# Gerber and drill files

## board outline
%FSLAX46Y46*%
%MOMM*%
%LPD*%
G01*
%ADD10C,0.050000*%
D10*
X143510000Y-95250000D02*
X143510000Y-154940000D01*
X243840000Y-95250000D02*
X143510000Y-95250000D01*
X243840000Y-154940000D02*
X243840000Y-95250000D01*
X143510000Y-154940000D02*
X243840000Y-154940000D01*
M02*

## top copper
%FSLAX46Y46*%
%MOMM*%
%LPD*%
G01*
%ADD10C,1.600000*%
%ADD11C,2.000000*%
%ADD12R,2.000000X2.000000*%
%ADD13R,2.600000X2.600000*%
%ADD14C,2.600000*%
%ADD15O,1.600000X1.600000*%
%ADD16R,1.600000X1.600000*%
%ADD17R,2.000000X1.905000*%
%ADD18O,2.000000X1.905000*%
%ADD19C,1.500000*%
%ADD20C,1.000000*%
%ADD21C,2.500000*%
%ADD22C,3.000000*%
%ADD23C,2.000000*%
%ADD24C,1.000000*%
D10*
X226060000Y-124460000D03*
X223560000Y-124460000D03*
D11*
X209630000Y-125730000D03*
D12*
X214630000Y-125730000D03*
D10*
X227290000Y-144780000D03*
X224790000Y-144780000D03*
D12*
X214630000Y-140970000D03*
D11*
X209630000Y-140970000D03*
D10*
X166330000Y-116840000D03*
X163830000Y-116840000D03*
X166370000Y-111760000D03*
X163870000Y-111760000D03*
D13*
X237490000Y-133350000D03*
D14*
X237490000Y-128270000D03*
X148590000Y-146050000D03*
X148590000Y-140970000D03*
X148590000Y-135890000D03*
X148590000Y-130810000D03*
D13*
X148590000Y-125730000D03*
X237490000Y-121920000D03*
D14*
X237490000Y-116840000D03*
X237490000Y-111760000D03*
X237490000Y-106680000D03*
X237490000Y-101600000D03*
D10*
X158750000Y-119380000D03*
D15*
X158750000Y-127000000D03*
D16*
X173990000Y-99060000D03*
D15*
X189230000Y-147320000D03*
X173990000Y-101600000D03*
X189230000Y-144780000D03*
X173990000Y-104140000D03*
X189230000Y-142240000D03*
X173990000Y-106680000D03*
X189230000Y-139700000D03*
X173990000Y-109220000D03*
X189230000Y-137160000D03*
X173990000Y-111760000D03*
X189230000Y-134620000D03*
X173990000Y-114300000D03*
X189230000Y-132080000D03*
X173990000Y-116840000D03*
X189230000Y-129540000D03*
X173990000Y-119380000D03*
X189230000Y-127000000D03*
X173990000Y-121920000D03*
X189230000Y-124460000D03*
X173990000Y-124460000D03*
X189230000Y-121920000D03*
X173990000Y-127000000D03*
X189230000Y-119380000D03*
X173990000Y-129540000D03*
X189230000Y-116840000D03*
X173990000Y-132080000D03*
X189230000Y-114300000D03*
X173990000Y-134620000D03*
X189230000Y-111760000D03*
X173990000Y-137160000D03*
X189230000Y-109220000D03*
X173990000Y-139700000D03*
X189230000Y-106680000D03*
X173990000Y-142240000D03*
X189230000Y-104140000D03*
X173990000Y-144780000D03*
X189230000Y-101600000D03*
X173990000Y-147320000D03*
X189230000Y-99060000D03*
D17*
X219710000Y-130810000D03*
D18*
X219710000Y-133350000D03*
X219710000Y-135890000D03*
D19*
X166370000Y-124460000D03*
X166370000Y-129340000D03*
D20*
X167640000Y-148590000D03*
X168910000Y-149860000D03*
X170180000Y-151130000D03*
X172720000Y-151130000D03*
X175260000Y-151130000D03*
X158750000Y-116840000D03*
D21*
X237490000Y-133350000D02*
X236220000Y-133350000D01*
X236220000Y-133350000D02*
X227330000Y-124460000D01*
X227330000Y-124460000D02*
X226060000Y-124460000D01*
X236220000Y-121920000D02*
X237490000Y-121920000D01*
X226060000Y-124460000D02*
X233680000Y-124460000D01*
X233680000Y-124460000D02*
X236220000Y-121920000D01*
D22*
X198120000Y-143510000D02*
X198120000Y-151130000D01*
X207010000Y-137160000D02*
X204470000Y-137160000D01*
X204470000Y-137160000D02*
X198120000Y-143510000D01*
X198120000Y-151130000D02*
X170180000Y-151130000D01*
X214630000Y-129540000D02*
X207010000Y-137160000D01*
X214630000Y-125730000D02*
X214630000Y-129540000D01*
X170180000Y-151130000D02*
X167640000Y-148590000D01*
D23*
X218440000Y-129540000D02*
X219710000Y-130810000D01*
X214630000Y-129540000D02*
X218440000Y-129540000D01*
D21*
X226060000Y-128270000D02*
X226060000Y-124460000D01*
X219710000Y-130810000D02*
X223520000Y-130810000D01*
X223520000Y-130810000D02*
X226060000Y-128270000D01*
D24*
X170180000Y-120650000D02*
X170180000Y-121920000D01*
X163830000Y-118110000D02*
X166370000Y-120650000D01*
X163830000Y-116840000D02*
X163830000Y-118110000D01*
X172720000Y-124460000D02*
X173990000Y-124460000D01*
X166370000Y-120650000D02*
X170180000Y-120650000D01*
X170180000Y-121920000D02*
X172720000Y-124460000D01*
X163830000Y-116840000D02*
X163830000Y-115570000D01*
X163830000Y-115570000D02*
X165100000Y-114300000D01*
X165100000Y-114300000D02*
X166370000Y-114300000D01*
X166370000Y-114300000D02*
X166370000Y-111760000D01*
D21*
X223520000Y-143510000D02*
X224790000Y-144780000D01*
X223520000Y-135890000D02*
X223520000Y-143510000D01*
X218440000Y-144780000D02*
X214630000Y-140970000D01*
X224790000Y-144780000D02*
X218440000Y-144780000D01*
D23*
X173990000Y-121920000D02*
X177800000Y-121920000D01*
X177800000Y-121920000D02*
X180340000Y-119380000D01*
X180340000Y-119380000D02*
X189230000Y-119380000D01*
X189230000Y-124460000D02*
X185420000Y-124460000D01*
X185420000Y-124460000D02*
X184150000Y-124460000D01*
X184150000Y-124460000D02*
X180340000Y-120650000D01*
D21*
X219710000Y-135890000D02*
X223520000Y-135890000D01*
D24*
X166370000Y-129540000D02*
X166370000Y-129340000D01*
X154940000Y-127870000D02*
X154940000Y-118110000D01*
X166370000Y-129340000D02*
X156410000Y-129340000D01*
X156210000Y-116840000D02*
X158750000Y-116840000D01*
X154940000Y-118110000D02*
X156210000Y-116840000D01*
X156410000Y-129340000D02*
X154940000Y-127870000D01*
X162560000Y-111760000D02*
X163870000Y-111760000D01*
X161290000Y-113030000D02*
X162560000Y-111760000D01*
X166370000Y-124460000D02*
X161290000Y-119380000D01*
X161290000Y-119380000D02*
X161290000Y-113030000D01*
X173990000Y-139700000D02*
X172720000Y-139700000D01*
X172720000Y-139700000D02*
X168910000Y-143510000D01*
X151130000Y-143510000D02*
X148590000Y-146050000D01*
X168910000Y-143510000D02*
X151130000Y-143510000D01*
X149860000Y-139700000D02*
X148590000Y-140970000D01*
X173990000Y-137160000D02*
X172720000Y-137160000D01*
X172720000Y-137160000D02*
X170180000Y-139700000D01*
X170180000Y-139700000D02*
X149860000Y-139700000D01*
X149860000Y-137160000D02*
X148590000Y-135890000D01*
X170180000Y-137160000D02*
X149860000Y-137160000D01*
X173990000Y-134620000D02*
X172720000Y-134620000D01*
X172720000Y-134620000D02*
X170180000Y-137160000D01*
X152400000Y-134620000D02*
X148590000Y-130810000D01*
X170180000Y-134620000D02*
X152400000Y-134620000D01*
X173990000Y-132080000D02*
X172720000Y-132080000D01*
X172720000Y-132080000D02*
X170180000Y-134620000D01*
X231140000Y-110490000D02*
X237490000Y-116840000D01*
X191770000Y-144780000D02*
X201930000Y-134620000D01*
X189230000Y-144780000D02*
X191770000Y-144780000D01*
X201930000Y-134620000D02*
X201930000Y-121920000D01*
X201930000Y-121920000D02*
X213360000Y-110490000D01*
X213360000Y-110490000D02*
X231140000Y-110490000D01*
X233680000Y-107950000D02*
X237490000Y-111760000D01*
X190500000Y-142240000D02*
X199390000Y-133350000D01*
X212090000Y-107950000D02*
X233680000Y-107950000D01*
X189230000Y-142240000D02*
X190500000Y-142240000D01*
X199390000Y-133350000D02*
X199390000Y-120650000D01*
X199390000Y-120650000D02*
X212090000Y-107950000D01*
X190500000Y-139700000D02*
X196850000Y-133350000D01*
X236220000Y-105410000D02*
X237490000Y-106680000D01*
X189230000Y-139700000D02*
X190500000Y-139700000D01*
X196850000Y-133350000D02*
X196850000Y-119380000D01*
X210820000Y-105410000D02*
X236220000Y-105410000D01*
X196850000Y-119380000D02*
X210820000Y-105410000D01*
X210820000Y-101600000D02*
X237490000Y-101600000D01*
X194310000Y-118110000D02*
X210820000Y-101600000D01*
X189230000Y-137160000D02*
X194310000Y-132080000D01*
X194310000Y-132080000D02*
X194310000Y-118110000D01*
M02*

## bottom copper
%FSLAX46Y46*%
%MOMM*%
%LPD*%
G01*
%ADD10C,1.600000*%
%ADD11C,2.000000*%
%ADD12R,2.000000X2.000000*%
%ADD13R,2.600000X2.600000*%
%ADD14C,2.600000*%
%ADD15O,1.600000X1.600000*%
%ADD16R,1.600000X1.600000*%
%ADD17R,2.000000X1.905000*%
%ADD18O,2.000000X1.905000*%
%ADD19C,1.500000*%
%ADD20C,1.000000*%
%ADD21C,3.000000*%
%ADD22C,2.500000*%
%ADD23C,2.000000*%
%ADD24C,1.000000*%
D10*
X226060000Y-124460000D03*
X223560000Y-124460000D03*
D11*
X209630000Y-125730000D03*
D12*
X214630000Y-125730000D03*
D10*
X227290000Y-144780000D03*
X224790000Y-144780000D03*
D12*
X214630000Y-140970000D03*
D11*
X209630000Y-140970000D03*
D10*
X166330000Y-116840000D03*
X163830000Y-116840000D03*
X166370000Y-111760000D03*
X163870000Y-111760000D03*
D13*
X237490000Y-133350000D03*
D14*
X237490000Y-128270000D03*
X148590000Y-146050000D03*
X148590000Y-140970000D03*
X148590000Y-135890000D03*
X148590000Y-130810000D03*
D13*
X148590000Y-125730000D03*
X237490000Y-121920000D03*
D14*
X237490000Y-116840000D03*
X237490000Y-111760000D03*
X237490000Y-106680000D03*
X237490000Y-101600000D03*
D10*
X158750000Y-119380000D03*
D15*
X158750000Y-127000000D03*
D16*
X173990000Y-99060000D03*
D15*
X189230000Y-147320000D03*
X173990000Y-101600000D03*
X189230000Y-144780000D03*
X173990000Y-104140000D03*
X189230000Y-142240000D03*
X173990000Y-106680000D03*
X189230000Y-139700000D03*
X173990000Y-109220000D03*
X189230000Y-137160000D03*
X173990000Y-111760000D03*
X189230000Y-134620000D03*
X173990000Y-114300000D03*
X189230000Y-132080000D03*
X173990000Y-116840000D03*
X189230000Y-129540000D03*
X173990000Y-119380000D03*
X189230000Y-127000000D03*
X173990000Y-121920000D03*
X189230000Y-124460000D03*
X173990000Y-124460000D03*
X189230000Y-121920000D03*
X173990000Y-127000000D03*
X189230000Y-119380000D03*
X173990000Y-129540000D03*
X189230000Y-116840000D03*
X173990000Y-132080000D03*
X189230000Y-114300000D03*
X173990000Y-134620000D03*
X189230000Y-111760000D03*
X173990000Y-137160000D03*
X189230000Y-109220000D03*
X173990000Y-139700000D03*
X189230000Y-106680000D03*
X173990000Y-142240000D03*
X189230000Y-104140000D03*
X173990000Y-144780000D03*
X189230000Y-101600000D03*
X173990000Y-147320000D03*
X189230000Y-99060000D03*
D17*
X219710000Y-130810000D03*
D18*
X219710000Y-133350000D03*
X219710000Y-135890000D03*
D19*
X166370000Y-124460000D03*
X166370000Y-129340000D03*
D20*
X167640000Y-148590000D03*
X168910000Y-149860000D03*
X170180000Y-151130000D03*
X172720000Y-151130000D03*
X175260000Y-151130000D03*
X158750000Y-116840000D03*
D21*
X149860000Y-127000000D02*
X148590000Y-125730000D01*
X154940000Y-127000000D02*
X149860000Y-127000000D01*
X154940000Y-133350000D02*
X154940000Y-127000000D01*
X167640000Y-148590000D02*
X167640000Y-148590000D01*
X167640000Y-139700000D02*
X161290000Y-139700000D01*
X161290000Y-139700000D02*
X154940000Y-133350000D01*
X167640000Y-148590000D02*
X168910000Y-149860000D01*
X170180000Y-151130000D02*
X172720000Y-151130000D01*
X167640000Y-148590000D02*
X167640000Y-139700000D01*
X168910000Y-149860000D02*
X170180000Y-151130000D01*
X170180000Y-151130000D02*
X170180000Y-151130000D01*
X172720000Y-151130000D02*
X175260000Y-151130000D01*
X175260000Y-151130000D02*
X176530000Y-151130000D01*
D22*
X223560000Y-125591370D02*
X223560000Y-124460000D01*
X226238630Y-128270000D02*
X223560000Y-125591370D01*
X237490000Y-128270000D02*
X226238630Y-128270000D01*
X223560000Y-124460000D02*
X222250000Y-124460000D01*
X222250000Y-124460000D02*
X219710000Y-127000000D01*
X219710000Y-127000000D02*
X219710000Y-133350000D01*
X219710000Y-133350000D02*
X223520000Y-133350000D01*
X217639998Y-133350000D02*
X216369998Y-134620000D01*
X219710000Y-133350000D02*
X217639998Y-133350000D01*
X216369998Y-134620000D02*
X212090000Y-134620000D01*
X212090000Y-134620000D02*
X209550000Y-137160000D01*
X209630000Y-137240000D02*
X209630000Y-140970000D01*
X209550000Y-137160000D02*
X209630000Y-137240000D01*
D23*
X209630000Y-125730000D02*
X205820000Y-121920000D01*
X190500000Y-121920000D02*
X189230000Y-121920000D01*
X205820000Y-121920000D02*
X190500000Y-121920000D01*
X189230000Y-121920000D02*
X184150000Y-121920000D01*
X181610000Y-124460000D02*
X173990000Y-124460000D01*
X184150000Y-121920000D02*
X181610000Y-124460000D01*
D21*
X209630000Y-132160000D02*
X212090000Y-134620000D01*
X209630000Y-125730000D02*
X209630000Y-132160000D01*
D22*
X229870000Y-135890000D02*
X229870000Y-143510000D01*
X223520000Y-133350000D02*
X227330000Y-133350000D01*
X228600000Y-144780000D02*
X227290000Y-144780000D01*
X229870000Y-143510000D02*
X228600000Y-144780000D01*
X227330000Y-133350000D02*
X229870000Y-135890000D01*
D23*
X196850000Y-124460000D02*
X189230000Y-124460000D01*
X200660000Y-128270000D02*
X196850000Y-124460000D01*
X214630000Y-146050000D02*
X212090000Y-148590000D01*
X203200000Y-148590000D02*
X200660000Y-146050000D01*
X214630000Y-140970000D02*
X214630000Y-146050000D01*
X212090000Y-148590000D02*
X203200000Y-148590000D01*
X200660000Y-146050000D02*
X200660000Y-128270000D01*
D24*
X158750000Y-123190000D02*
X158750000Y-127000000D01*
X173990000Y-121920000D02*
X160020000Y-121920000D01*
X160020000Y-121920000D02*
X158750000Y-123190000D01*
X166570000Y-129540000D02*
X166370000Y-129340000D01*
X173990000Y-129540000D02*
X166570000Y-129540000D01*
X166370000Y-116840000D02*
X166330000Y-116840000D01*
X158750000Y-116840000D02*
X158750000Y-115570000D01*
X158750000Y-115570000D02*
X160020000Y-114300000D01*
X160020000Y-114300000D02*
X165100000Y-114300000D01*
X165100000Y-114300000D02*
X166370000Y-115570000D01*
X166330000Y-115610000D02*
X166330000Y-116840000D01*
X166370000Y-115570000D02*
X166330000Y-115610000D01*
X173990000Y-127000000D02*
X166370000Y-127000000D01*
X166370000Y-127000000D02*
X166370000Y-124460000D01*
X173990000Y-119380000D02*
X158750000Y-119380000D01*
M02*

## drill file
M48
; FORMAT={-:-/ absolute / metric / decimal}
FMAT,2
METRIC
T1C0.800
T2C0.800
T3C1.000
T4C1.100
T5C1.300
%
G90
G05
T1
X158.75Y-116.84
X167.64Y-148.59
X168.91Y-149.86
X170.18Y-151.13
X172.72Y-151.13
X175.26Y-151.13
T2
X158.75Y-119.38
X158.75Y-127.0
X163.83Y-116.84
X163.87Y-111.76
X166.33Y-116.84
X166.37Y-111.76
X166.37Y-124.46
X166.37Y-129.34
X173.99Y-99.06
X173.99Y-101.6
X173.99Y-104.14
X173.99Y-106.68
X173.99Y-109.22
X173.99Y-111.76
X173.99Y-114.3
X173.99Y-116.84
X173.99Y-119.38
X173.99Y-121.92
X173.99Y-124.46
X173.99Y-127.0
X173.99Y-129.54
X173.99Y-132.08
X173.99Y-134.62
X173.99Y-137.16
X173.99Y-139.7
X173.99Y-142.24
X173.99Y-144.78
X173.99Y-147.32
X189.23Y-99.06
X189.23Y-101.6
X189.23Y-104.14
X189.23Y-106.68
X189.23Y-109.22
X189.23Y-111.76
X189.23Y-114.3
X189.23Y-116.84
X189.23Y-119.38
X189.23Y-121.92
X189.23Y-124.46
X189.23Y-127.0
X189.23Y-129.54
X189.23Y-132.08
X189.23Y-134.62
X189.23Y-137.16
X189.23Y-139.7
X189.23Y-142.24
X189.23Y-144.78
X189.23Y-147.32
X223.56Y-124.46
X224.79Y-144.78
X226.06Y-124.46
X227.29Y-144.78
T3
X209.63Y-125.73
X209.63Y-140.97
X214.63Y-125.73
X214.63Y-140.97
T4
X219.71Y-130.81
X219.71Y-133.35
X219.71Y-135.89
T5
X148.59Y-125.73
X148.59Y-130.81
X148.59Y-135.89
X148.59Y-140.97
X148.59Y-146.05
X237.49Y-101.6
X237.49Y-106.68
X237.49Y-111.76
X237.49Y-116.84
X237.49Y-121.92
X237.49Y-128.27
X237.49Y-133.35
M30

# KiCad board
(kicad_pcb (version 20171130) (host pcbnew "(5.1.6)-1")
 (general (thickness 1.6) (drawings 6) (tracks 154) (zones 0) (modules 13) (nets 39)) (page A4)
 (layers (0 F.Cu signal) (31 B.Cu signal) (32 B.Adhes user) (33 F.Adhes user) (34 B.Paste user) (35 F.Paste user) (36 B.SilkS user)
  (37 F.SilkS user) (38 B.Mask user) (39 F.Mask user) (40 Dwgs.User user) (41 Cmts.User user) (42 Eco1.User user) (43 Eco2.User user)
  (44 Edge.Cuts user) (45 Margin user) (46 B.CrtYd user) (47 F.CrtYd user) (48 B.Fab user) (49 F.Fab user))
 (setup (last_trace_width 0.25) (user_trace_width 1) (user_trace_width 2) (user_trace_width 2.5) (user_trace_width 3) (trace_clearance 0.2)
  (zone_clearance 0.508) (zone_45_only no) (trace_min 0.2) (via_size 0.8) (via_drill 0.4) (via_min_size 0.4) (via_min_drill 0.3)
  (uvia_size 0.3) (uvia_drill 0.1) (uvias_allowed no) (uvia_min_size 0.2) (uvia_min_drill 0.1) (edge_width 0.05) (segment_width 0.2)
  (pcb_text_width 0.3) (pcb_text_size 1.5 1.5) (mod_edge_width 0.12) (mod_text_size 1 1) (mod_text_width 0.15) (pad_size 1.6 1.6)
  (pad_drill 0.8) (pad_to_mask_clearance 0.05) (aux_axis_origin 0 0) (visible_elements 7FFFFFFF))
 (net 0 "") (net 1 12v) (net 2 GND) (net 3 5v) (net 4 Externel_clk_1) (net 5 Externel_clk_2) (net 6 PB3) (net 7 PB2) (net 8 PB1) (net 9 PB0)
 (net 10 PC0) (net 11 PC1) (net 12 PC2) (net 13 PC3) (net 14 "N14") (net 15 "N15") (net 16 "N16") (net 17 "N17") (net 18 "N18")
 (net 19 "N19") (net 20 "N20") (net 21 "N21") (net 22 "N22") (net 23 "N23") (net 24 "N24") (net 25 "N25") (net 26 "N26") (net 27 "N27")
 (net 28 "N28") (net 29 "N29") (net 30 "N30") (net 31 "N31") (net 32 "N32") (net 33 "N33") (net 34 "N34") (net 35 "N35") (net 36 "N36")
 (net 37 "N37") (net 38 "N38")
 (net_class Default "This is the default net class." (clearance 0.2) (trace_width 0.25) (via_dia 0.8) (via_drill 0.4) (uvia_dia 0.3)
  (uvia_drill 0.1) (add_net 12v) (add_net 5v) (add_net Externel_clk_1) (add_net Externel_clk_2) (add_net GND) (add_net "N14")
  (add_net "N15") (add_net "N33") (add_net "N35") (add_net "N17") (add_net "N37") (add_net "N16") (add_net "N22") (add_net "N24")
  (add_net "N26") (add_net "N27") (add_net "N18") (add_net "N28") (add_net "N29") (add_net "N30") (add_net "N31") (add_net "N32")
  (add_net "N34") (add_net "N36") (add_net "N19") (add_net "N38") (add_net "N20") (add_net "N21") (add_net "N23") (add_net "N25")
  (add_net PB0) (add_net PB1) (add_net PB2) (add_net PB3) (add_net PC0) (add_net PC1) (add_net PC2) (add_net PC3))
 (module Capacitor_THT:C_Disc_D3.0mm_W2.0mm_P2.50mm (layer F.Cu) (at 226.06 124.46 180)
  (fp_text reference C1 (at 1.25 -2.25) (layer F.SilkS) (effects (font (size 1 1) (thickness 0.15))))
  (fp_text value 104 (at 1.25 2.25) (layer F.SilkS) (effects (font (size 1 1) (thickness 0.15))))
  (pad 1 thru_hole circle (at 0 0 180) (size 1.6 1.6) (drill 0.8) (layers *.Cu *.Mask) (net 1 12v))
  (pad 2 thru_hole circle (at 2.5 0 180) (size 1.6 1.6) (drill 0.8) (layers *.Cu *.Mask) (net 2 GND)))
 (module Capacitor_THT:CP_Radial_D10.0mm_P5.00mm (layer F.Cu) (at 214.63 125.73 180)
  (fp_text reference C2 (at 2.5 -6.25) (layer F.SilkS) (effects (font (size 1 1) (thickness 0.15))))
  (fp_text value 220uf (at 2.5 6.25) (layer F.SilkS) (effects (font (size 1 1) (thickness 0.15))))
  (pad 2 thru_hole circle (at 5 0 180) (size 2 2) (drill 1) (layers *.Cu *.Mask) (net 2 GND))
  (pad 1 thru_hole rect (at 0 0 180) (size 2 2) (drill 1) (layers *.Cu *.Mask) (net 1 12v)))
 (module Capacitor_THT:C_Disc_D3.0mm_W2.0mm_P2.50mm (layer F.Cu) (at 224.79 144.78)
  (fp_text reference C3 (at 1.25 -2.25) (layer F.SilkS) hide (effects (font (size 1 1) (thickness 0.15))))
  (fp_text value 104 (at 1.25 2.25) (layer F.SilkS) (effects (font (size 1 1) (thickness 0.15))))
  (pad 2 thru_hole circle (at 2.5 0) (size 1.6 1.6) (drill 0.8) (layers *.Cu *.Mask) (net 2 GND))
  (pad 1 thru_hole circle (at 0 0) (size 1.6 1.6) (drill 0.8) (layers *.Cu *.Mask) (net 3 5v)))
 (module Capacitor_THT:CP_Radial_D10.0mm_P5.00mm (layer F.Cu) (at 214.63 140.97 180)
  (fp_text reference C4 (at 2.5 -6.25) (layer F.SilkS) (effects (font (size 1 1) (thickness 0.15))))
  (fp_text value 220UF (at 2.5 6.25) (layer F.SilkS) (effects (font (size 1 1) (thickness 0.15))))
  (pad 1 thru_hole rect (at 0 0 180) (size 2 2) (drill 1) (layers *.Cu *.Mask) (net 3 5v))
  (pad m2 thru_hole circle (at 5 0 180) (size 2 2) (drill 1) (layers *.Cu *.Mask) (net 2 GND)))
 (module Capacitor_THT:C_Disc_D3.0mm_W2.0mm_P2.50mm (layer F.Cu) (at 163.83 116.84)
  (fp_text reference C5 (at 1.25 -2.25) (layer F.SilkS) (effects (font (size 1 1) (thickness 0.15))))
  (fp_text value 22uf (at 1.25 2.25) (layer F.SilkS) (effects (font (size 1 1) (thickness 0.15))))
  (pad 2 thru_hole circle (at 2.5 0) (size 1.6 1.6) (drill 0.8) (layers *.Cu *.Mask) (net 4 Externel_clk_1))
  (pad 1 thru_hole circle (at 0 0) (size 1.6 1.6) (drill 0.8) (layers *.Cu *.Mask) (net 2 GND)))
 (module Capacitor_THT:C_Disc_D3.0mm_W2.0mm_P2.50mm (layer F.Cu) (at 166.37 111.76 180)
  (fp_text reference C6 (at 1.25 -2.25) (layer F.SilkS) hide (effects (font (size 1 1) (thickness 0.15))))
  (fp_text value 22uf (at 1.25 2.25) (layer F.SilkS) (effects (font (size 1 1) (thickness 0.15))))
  (pad 1 thru_hole circle (at 0 0 180) (size 1.6 1.6) (drill 0.8) (layers *.Cu *.Mask) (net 2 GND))
  (pad 2 thru_hole circle (at 2.5 0 180) (size 1.6 1.6) (drill 0.8) (layers *.Cu *.Mask) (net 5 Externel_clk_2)))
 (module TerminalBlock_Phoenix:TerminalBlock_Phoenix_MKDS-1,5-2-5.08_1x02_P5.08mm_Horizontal (layer F.Cu) (at 237.49 133.35 90)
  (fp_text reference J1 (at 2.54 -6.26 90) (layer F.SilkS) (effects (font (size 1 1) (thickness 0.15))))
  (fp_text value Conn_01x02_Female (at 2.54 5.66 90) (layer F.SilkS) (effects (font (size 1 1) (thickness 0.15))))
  (pad 1 thru_hole rect (at 0 0 90) (size 2.6 2.6) (drill 1.3) (layers *.Cu *.Mask) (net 1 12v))
  (pad 2 thru_hole circle (at 5.08 0 90) (size 2.6 2.6) (drill 1.3) (layers *.Cu *.Mask) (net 2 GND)))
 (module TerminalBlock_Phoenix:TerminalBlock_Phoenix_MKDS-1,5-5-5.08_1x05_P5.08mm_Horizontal (layer F.Cu) (at 148.59 125.73 270)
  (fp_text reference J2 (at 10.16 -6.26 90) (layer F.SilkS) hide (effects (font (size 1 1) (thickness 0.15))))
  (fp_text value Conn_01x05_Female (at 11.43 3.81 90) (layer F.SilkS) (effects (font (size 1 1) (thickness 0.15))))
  (pad 5 thru_hole circle (at 20.32 0 270) (size 2.6 2.6) (drill 1.3) (layers *.Cu *.Mask) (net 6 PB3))
  (pad 4 thru_hole circle (at 15.24 0 270) (size 2.6 2.6) (drill 1.3) (layers *.Cu *.Mask) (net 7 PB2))
  (pad 3 thru_hole circle (at 10.16 0 270) (size 2.6 2.6) (drill 1.3) (layers *.Cu *.Mask) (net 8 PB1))
  (pad 2 thru_hole circle (at 5.08 0 270) (size 2.6 2.6) (drill 1.3) (layers *.Cu *.Mask) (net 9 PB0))
  (pad 1 thru_hole rect (at 0 0 270) (size 2.6 2.6) (drill 1.3) (layers *.Cu *.Mask) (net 1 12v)))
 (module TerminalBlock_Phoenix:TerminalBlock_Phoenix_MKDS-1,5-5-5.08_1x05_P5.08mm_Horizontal (layer F.Cu) (at 237.49 121.92 90)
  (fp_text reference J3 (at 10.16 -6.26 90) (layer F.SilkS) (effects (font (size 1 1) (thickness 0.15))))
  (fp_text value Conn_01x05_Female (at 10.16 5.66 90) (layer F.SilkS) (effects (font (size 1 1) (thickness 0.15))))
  (pad 1 thru_hole rect (at 0 0 90) (size 2.6 2.6) (drill 1.3) (layers *.Cu *.Mask) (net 1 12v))
  (pad 2 thru_hole circle (at 5.08 0 90) (size 2.6 2.6) (drill 1.3) (layers *.Cu *.Mask) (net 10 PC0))
  (pad 3 thru_hole circle (at 10.16 0 90) (size 2.6 2.6) (drill 1.3) (layers *.Cu *.Mask) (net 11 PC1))
  (pad 4 thru_hole circle (at 15.24 0 90) (size 2.6 2.6) (drill 1.3) (layers *.Cu *.Mask) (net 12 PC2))
  (pad 5 thru_hole circle (at 20.32 0 90) (size 2.6 2.6) (drill 1.3) (layers *.Cu *.Mask) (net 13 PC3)))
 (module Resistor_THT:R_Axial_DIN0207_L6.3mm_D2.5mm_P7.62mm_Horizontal (layer F.Cu) (at 158.75 119.38 270)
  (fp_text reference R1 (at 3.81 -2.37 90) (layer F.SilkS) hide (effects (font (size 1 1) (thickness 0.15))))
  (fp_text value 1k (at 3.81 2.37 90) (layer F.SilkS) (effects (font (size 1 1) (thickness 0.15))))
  (pad 1 thru_hole circle (at 0 0 270) (size 1.6 1.6) (drill 0.8) (layers *.Cu *.Mask) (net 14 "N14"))
  (pad 2 thru_hole oval (at 7.62 0 270) (size 1.6 1.6) (drill 0.8) (layers *.Cu *.Mask) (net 3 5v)))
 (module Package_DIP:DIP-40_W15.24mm (layer F.Cu) (at 173.99 99.06)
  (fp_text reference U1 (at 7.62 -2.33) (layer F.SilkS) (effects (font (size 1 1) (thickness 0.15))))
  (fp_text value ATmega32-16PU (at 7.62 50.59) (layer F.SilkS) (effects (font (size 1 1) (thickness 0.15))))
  (pad 1 thru_hole rect (at 0 0) (size 1.6 1.6) (drill 0.8) (layers *.Cu *.Mask) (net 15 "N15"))
  (pad 21 thru_hole oval (at 15.24 48.26) (size 1.6 1.6) (drill 0.8) (layers *.Cu *.Mask) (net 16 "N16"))
  (pad 2 thru_hole oval (at 0 2.54) (size 1.6 1.6) (drill 0.8) (layers *.Cu *.Mask) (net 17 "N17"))
  (pad 22 thru_hole oval (at 15.24 45.72) (size 1.6 1.6) (drill 0.8) (layers *.Cu *.Mask) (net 10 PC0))
  (pad 3 thru_hole oval (at 0 5.08) (size 1.6 1.6) (drill 0.8) (layers *.Cu *.Mask) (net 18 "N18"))
  (pad 23 thru_hole oval (at 15.24 43.18) (size 1.6 1.6) (drill 0.8) (layers *.Cu *.Mask) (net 11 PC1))
  (pad 4 thru_hole oval (at 0 7.62) (size 1.6 1.6) (drill 0.8) (layers *.Cu *.Mask) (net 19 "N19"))
  (pad 24 thru_hole oval (at 15.24 40.64) (size 1.6 1.6) (drill 0.8) (layers *.Cu *.Mask) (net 12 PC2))
  (pad 5 thru_hole oval (at 0 10.16) (size 1.6 1.6) (drill 0.8) (layers *.Cu *.Mask) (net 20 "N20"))
  (pad 25 thru_hole oval (at 15.24 38.1) (size 1.6 1.6) (drill 0.8) (layers *.Cu *.Mask) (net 13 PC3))
  (pad 6 thru_hole oval (at 0 12.7) (size 1.6 1.6) (drill 0.8) (layers *.Cu *.Mask) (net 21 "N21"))
  (pad 26 thru_hole oval (at 15.24 35.56) (size 1.6 1.6) (drill 0.8) (layers *.Cu *.Mask) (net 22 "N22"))
  (pad 7 thru_hole oval (at 0 15.24) (size 1.6 1.6) (drill 0.8) (layers *.Cu *.Mask) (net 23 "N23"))
  (pad 27 thru_hole oval (at 15.24 33.02) (size 1.6 1.6) (drill 0.8) (layers *.Cu *.Mask) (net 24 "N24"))
  (pad 8 thru_hole oval (at 0 17.78) (size 1.6 1.6) (drill 0.8) (layers *.Cu *.Mask) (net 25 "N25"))
  (pad 28 thru_hole oval (at 15.24 30.48) (size 1.6 1.6) (drill 0.8) (layers *.Cu *.Mask) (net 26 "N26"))
  (pad 9 thru_hole oval (at 0 20.32) (size 1.6 1.6) (drill 0.8) (layers *.Cu *.Mask) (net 14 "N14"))
  (pad 29 thru_hole oval (at 15.24 27.94) (size 1.6 1.6) (drill 0.8) (layers *.Cu *.Mask) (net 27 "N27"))
  (pad 10 thru_hole oval (at 0 22.86) (size 1.6 1.6) (drill 0.8) (layers *.Cu *.Mask) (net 3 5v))
  (pad 30 thru_hole oval (at 15.24 25.4) (size 1.6 1.6) (drill 0.8) (layers *.Cu *.Mask) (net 3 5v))
  (pad 11 thru_hole oval (at 0 25.4) (size 1.6 1.6) (drill 0.8) (layers *.Cu *.Mask) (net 2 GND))
  (pad 31 thru_hole oval (at 15.24 22.86) (size 1.6 1.6) (drill 0.8) (layers *.Cu *.Mask) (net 2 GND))
  (pad 12 thru_hole oval (at 0 27.94) (size 1.6 1.6) (drill 0.8) (layers *.Cu *.Mask) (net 5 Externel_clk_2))
  (pad 32 thru_hole oval (at 15.24 20.32) (size 1.6 1.6) (drill 0.8) (layers *.Cu *.Mask) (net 3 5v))
  (pad 13 thru_hole oval (at 0 30.48) (size 1.6 1.6) (drill 0.8) (layers *.Cu *.Mask) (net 4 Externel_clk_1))
  (pad 33 thru_hole oval (at 15.24 17.78) (size 1.6 1.6) (drill 0.8) (layers *.Cu *.Mask) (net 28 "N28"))
  (pad 14 thru_hole oval (at 0 33.02) (size 1.6 1.6) (drill 0.8) (layers *.Cu *.Mask) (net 9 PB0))
  (pad 34 thru_hole oval (at 15.24 15.24) (size 1.6 1.6) (drill 0.8) (layers *.Cu *.Mask) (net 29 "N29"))
  (pad 15 thru_hole oval (at 0 35.56) (size 1.6 1.6) (drill 0.8) (layers *.Cu *.Mask) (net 8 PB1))
  (pad 35 thru_hole oval (at 15.24 12.7) (size 1.6 1.6) (drill 0.8) (layers *.Cu *.Mask) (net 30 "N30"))
  (pad 16 thru_hole oval (at 0 38.1) (size 1.6 1.6) (drill 0.8) (layers *.Cu *.Mask) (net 7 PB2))
  (pad 36 thru_hole oval (at 15.24 10.16) (size 1.6 1.6) (drill 0.8) (layers *.Cu *.Mask) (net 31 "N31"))
  (pad 17 thru_hole oval (at 0 40.64) (size 1.6 1.6) (drill 0.8) (layers *.Cu *.Mask) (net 6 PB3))
  (pad 37 thru_hole oval (at 15.24 7.62) (size 1.6 1.6) (drill 0.8) (layers *.Cu *.Mask) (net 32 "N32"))
  (pad 18 thru_hole oval (at 0 43.18) (size 1.6 1.6) (drill 0.8) (layers *.Cu *.Mask) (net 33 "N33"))
  (pad 38 thru_hole oval (at 15.24 5.08) (size 1.6 1.6) (drill 0.8) (layers *.Cu *.Mask) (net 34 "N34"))
  (pad 19 thru_hole oval (at 0 45.72) (size 1.6 1.6) (drill 0.8) (layers *.Cu *.Mask) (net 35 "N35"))
  (pad 39 thru_hole oval (at 15.24 2.54) (size 1.6 1.6) (drill 0.8) (layers *.Cu *.Mask) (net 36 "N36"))
  (pad 20 thru_hole oval (at 0 48.26) (size 1.6 1.6) (drill 0.8) (layers *.Cu *.Mask) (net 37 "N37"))
  (pad 40 thru_hole oval (at 15.24 0) (size 1.6 1.6) (drill 0.8) (layers *.Cu *.Mask) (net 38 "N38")))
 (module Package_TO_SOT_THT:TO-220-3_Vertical (layer F.Cu) (at 219.71 130.81 270)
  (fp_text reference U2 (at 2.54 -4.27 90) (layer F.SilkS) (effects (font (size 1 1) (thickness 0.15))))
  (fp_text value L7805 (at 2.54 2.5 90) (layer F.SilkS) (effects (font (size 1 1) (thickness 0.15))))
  (pad 1 thru_hole rect (at 0 0 270) (size 1.905 2) (drill 1.1) (layers *.Cu *.Mask) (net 1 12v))
  (pad 2 thru_hole oval (at 2.54 0 270) (size 1.905 2) (drill 1.1) (layers *.Cu *.Mask) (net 2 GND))
  (pad 3 thru_hole oval (at 5.08 0 270) (size 1.905 2) (drill 1.1) (layers *.Cu *.Mask) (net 3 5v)))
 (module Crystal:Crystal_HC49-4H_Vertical (layer F.Cu) (at 166.37 124.46 270)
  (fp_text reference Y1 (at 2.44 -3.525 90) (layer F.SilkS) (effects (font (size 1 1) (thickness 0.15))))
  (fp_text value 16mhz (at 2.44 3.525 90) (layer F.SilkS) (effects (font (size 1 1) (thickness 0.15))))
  (pad 1 thru_hole circle (at 0 0 270) (size 1.5 1.5) (drill 0.8) (layers *.Cu *.Mask) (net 5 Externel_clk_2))
  (pad 2 thru_hole circle (at 4.88 0 270) (size 1.5 1.5) (drill 0.8) (layers *.Cu *.Mask) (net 4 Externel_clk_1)))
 (gr_line (start 143.51 95.25) (end 143.51 154.94) (layer Edge.Cuts) (width 0.05))
 (gr_line (start 243.84 95.25) (end 143.51 95.25) (layer Edge.Cuts) (width 0.05))
 (gr_line (start 243.84 154.94) (end 243.84 95.25) (layer Edge.Cuts) (width 0.05))
 (gr_line (start 143.51 154.94) (end 243.84 154.94) (layer Edge.Cuts) (width 0.05))
 (segment (start 237.49 133.35) (end 236.22 133.35) (width 2.5) (layer F.Cu) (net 1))
 (segment (start 236.22 133.35) (end 227.33 124.46) (width 2.5) (layer F.Cu) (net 1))
 (segment (start 227.33 124.46) (end 226.06 124.46) (width 2.5) (layer F.Cu) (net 1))
 (segment (start 236.22 121.92) (end 237.49 121.92) (width 2.5) (layer F.Cu) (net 1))
 (segment (start 226.06 124.46) (end 233.68 124.46) (width 2.5) (layer F.Cu) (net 1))
 (segment (start 233.68 124.46) (end 236.22 121.92) (width 2.5) (layer F.Cu) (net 1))
 (segment (start 149.86 127) (end 148.59 125.73) (width 3) (layer B.Cu) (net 1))
 (segment (start 154.94 127) (end 149.86 127) (width 3) (layer B.Cu) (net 1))
 (segment (start 198.12 143.51) (end 198.12 151.13) (width 3) (layer F.Cu) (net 1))
 (segment (start 207.01 137.16) (end 204.47 137.16) (width 3) (layer F.Cu) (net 1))
 (segment (start 204.47 137.16) (end 198.12 143.51) (width 3) (layer F.Cu) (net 1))
 (segment (start 198.12 151.13) (end 170.18 151.13) (width 3) (layer F.Cu) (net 1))
 (segment (start 214.63 129.54) (end 207.01 137.16) (width 3) (layer F.Cu) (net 1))
 (segment (start 154.94 133.35) (end 154.94 127) (width 3) (layer B.Cu) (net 1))
 (segment (start 214.63 125.73) (end 214.63 129.54) (width 3) (layer F.Cu) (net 1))
 (segment (start 170.18 151.13) (end 167.64 148.59) (width 3) (layer F.Cu) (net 1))
 (segment (start 167.64 148.59) (end 167.64 148.59) (width 3) (layer B.Cu) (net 1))
 (segment (start 167.64 139.7) (end 161.29 139.7) (width 3) (layer B.Cu) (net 1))
 (segment (start 161.29 139.7) (end 154.94 133.35) (width 3) (layer B.Cu) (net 1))
 (segment (start 167.64 148.59) (end 168.91 149.86) (width 3) (layer B.Cu) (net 1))
 (segment (start 170.18 151.13) (end 172.72 151.13) (width 3) (layer B.Cu) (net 1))
 (segment (start 167.64 148.59) (end 167.64 139.7) (width 3) (layer B.Cu) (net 1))
 (via (at 167.64 148.59) (size 1) (drill 0.8) (layers F.Cu B.Cu) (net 1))
 (segment (start 168.91 149.86) (end 170.18 151.13) (width 3) (layer B.Cu) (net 1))
 (via (at 168.91 149.86) (size 1) (drill 0.8) (layers F.Cu B.Cu) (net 1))
 (segment (start 170.18 151.13) (end 170.18 151.13) (width 3) (layer B.Cu) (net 1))
 (via (at 170.18 151.13) (size 1) (drill 0.8) (layers F.Cu B.Cu) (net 1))
 (segment (start 172.72 151.13) (end 175.26 151.13) (width 3) (layer B.Cu) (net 1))
 (via (at 172.72 151.13) (size 1) (drill 0.8) (layers F.Cu B.Cu) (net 1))
 (segment (start 175.26 151.13) (end 176.53 151.13) (width 3) (layer B.Cu) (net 1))
 (via (at 175.26 151.13) (size 1) (drill 0.8) (layers F.Cu B.Cu) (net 1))
 (segment (start 218.44 129.54) (end 219.71 130.81) (width 2) (layer F.Cu) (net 1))
 (segment (start 214.63 129.54) (end 218.44 129.54) (width 2) (layer F.Cu) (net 1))
 (segment (start 226.06 128.27) (end 226.06 124.46) (width 2.5) (layer F.Cu) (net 1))
 (segment (start 219.71 130.81) (end 223.52 130.81) (width 2.5) (layer F.Cu) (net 1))
 (segment (start 223.52 130.81) (end 226.06 128.27) (width 2.5) (layer F.Cu) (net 1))
 (segment (start 223.56 125.59137) (end 223.56 124.46) (width 2.5) (layer B.Cu) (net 2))
 (segment (start 226.23863 128.27) (end 223.56 125.59137) (width 2.5) (layer B.Cu) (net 2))
 (segment (start 237.49 128.27) (end 226.23863 128.27) (width 2.5) (layer B.Cu) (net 2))
 (segment (start 223.56 124.46) (end 222.25 124.46) (width 2.5) (layer B.Cu) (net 2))
 (segment (start 222.25 124.46) (end 219.71 127) (width 2.5) (layer B.Cu) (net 2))
 (segment (start 219.71 127) (end 219.71 133.35) (width 2.5) (layer B.Cu) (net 2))
 (segment (start 219.71 133.35) (end 223.52 133.35) (width 2.5) (layer B.Cu) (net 2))
 (segment (start 217.639998 133.35) (end 216.369998 134.62) (width 2.5) (layer B.Cu) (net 2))
 (segment (start 219.71 133.35) (end 217.639998 133.35) (width 2.5) (layer B.Cu) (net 2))
 (segment (start 216.369998 134.62) (end 212.09 134.62) (width 2.5) (layer B.Cu) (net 2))
 (segment (start 212.09 134.62) (end 209.55 137.16) (width 2.5) (layer B.Cu) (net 2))
 (segment (start 209.63 137.24) (end 209.63 140.97) (width 2.5) (layer B.Cu) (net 2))
 (segment (start 209.55 137.16) (end 209.63 137.24) (width 2.5) (layer B.Cu) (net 2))
 (segment (start 209.63 125.73) (end 205.82 121.92) (width 2) (layer B.Cu) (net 2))
 (segment (start 190.5 121.92) (end 189.23 121.92) (width 2) (layer B.Cu) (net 2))
 (segment (start 205.82 121.92) (end 190.5 121.92) (width 2) (layer B.Cu) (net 2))
 (segment (start 189.23 121.92) (end 184.15 121.92) (width 2) (layer B.Cu) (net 2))
 (segment (start 181.61 124.46) (end 173.99 124.46) (width 2) (layer B.Cu) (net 2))
 (segment (start 184.15 121.92) (end 181.61 124.46) (width 2) (layer B.Cu) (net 2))
 (segment (start 209.63 132.16) (end 212.09 134.62) (width 3) (layer B.Cu) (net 2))
 (segment (start 209.63 125.73) (end 209.63 132.16) (width 3) (layer B.Cu) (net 2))
 (segment (start 229.87 135.89) (end 229.87 143.51) (width 2.5) (layer B.Cu) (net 2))
 (segment (start 223.52 133.35) (end 227.33 133.35) (width 2.5) (layer B.Cu) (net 2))
 (segment (start 228.6 144.78) (end 227.29 144.78) (width 2.5) (layer B.Cu) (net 2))
 (segment (start 229.87 143.51) (end 228.6 144.78) (width 2.5) (layer B.Cu) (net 2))
 (segment (start 227.33 133.35) (end 229.87 135.89) (width 2.5) (layer B.Cu) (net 2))
 (segment (start 170.18 120.65) (end 170.18 121.92) (width 1) (layer F.Cu) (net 2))
 (segment (start 163.83 118.11) (end 166.37 120.65) (width 1) (layer F.Cu) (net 2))
 (segment (start 163.83 116.84) (end 163.83 118.11) (width 1) (layer F.Cu) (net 2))
 (segment (start 172.72 124.46) (end 173.99 124.46) (width 1) (layer F.Cu) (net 2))
 (segment (start 166.37 120.65) (end 170.18 120.65) (width 1) (layer F.Cu) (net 2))
 (segment (start 170.18 121.92) (end 172.72 124.46) (width 1) (layer F.Cu) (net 2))
 (segment (start 163.83 116.84) (end 163.83 115.57) (width 1) (layer F.Cu) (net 2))
 (segment (start 163.83 115.57) (end 165.1 114.3) (width 1) (layer F.Cu) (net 2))
 (segment (start 165.1 114.3) (end 166.37 114.3) (width 1) (layer F.Cu) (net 2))
 (segment (start 166.37 114.3) (end 166.37 111.76) (width 1) (layer F.Cu) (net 2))
 (segment (start 223.52 143.51) (end 224.79 144.78) (width 2.5) (layer F.Cu) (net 3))
 (segment (start 223.52 135.89) (end 223.52 143.51) (width 2.5) (layer F.Cu) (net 3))
 (segment (start 218.44 144.78) (end 214.63 140.97) (width 2.5) (layer F.Cu) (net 3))
 (segment (start 224.79 144.78) (end 218.44 144.78) (width 2.5) (layer F.Cu) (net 3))
 (segment (start 196.85 124.46) (end 189.23 124.46) (width 2) (layer B.Cu) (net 3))
 (segment (start 200.66 128.27) (end 196.85 124.46) (width 2) (layer B.Cu) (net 3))
 (segment (start 214.63 146.05) (end 212.09 148.59) (width 2) (layer B.Cu) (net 3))
 (segment (start 203.2 148.59) (end 200.66 146.05) (width 2) (layer B.Cu) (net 3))
 (segment (start 214.63 140.97) (end 214.63 146.05) (width 2) (layer B.Cu) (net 3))
 (segment (start 212.09 148.59) (end 203.2 148.59) (width 2) (layer B.Cu) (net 3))
 (segment (start 200.66 146.05) (end 200.66 128.27) (width 2) (layer B.Cu) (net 3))
 (segment (start 173.99 121.92) (end 177.8 121.92) (width 2) (layer F.Cu) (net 3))
 (segment (start 177.8 121.92) (end 180.34 119.38) (width 2) (layer F.Cu) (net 3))
 (segment (start 158.75 123.19) (end 158.75 127) (width 1) (layer B.Cu) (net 3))
 (segment (start 173.99 121.92) (end 160.02 121.92) (width 1) (layer B.Cu) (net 3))
 (segment (start 160.02 121.92) (end 158.75 123.19) (width 1) (layer B.Cu) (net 3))
 (segment (start 180.34 119.38) (end 189.23 119.38) (width 2) (layer F.Cu) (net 3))
 (segment (start 189.23 124.46) (end 185.42 124.46) (width 2) (layer F.Cu) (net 3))
 (segment (start 185.42 124.46) (end 184.15 124.46) (width 2) (layer F.Cu) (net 3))
 (segment (start 184.15 124.46) (end 180.34 120.65) (width 2) (layer F.Cu) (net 3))
 (segment (start 219.71 135.89) (end 223.52 135.89) (width 2.5) (layer F.Cu) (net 3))
 (via (at 158.75 116.84) (size 1) (drill 0.8) (layers F.Cu B.Cu) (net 4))
 (segment (start 166.57 129.54) (end 166.37 129.34) (width 1) (layer B.Cu) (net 4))
 (segment (start 173.99 129.54) (end 166.57 129.54) (width 1) (layer B.Cu) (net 4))
 (segment (start 166.37 116.84) (end 166.33 116.84) (width 1) (layer B.Cu) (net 4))
 (segment (start 166.37 129.54) (end 166.37 129.34) (width 1) (layer F.Cu) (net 4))
 (segment (start 154.94 127.87) (end 154.94 118.11) (width 1) (layer F.Cu) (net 4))
 (segment (start 166.37 129.34) (end 156.41 129.34) (width 1) (layer F.Cu) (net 4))
 (segment (start 156.21 116.84) (end 158.75 116.84) (width 1) (layer F.Cu) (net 4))
 (segment (start 154.94 118.11) (end 156.21 116.84) (width 1) (layer F.Cu) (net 4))
 (segment (start 156.41 129.34) (end 154.94 127.87) (width 1) (layer F.Cu) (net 4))
 (segment (start 158.75 116.84) (end 158.75 115.57) (width 1) (layer B.Cu) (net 4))
 (segment (start 158.75 115.57) (end 160.02 114.3) (width 1) (layer B.Cu) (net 4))
 (segment (start 160.02 114.3) (end 165.1 114.3) (width 1) (layer B.Cu) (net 4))
 (segment (start 165.1 114.3) (end 166.37 115.57) (width 1) (layer B.Cu) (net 4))
 (segment (start 166.33 115.61) (end 166.33 116.84) (width 1) (layer B.Cu) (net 4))
 (segment (start 166.37 115.57) (end 166.33 115.61) (width 1) (layer B.Cu) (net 4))
 (segment (start 173.99 127) (end 166.37 127) (width 1) (layer B.Cu) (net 5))
 (segment (start 166.37 127) (end 166.37 124.46) (width 1) (layer B.Cu) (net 5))
 (segment (start 162.56 111.76) (end 163.87 111.76) (width 1) (layer F.Cu) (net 5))
 (segment (start 161.29 113.03) (end 162.56 111.76) (width 1) (layer F.Cu) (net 5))
 (segment (start 166.37 124.46) (end 161.29 119.38) (width 1) (layer F.Cu) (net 5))
 (segment (start 161.29 119.38) (end 161.29 113.03) (width 1) (layer F.Cu) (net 5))
 (segment (start 173.99 139.7) (end 172.72 139.7) (width 1) (layer F.Cu) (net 6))
 (segment (start 172.72 139.7) (end 168.91 143.51) (width 1) (layer F.Cu) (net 6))
 (segment (start 151.13 143.51) (end 148.59 146.05) (width 1) (layer F.Cu) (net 6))
 (segment (start 168.91 143.51) (end 151.13 143.51) (width 1) (layer F.Cu) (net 6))
 (segment (start 149.86 139.7) (end 148.59 140.97) (width 1) (layer F.Cu) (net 7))
 (segment (start 173.99 137.16) (end 172.72 137.16) (width 1) (layer F.Cu) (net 7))
 (segment (start 172.72 137.16) (end 170.18 139.7) (width 1) (layer F.Cu) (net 7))
 (segment (start 170.18 139.7) (end 149.86 139.7) (width 1) (layer F.Cu) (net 7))
 (segment (start 149.86 137.16) (end 148.59 135.89) (width 1) (layer F.Cu) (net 8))
 (segment (start 170.18 137.16) (end 149.86 137.16) (width 1) (layer F.Cu) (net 8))
 (segment (start 173.99 134.62) (end 172.72 134.62) (width 1) (layer F.Cu) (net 8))
 (segment (start 172.72 134.62) (end 170.18 137.16) (width 1) (layer F.Cu) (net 8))
 (segment (start 152.4 134.62) (end 148.59 130.81) (width 1) (layer F.Cu) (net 9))
 (segment (start 170.18 134.62) (end 152.4 134.62) (width 1) (layer F.Cu) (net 9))
 (segment (start 173.99 132.08) (end 172.72 132.08) (width 1) (layer F.Cu) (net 9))
 (segment (start 172.72 132.08) (end 170.18 134.62) (width 1) (layer F.Cu) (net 9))
 (segment (start 231.14 110.49) (end 237.49 116.84) (width 1) (layer F.Cu) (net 10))
 (segment (start 191.77 144.78) (end 201.93 134.62) (width 1) (layer F.Cu) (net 10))
 (segment (start 189.23 144.78) (end 191.77 144.78) (width 1) (layer F.Cu) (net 10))
 (segment (start 201.93 134.62) (end 201.93 121.92) (width 1) (layer F.Cu) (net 10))
 (segment (start 201.93 121.92) (end 213.36 110.49) (width 1) (layer F.Cu) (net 10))
 (segment (start 213.36 110.49) (end 231.14 110.49) (width 1) (layer F.Cu) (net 10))
 (segment (start 233.68 107.95) (end 237.49 111.76) (width 1) (layer F.Cu) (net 11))
 (segment (start 190.5 142.24) (end 199.39 133.35) (width 1) (layer F.Cu) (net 11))
 (segment (start 212.09 107.95) (end 233.68 107.95) (width 1) (layer F.Cu) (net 11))
 (segment (start 189.23 142.24) (end 190.5 142.24) (width 1) (layer F.Cu) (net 11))
 (segment (start 199.39 133.35) (end 199.39 120.65) (width 1) (layer F.Cu) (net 11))
 (segment (start 199.39 120.65) (end 212.09 107.95) (width 1) (layer F.Cu) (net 11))
 (segment (start 190.5 139.7) (end 196.85 133.35) (width 1) (layer F.Cu) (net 12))
 (segment (start 236.22 105.41) (end 237.49 106.68) (width 1) (layer F.Cu) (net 12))
 (segment (start 189.23 139.7) (end 190.5 139.7) (width 1) (layer F.Cu) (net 12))
 (segment (start 196.85 133.35) (end 196.85 119.38) (width 1) (layer F.Cu) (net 12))
 (segment (start 210.82 105.41) (end 236.22 105.41) (width 1) (layer F.Cu) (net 12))
 (segment (start 196.85 119.38) (end 210.82 105.41) (width 1) (layer F.Cu) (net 12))
 (segment (start 210.82 101.6) (end 237.49 101.6) (width 1) (layer F.Cu) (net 13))
 (segment (start 194.31 118.11) (end 210.82 101.6) (width 1) (layer F.Cu) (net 13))
 (segment (start 189.23 137.16) (end 194.31 132.08) (width 1) (layer F.Cu) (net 13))
 (segment (start 194.31 132.08) (end 194.31 118.11) (width 1) (layer F.Cu) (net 13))
 (segment (start 173.99 119.38) (end 158.75 119.38) (width 1) (layer B.Cu) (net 14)))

